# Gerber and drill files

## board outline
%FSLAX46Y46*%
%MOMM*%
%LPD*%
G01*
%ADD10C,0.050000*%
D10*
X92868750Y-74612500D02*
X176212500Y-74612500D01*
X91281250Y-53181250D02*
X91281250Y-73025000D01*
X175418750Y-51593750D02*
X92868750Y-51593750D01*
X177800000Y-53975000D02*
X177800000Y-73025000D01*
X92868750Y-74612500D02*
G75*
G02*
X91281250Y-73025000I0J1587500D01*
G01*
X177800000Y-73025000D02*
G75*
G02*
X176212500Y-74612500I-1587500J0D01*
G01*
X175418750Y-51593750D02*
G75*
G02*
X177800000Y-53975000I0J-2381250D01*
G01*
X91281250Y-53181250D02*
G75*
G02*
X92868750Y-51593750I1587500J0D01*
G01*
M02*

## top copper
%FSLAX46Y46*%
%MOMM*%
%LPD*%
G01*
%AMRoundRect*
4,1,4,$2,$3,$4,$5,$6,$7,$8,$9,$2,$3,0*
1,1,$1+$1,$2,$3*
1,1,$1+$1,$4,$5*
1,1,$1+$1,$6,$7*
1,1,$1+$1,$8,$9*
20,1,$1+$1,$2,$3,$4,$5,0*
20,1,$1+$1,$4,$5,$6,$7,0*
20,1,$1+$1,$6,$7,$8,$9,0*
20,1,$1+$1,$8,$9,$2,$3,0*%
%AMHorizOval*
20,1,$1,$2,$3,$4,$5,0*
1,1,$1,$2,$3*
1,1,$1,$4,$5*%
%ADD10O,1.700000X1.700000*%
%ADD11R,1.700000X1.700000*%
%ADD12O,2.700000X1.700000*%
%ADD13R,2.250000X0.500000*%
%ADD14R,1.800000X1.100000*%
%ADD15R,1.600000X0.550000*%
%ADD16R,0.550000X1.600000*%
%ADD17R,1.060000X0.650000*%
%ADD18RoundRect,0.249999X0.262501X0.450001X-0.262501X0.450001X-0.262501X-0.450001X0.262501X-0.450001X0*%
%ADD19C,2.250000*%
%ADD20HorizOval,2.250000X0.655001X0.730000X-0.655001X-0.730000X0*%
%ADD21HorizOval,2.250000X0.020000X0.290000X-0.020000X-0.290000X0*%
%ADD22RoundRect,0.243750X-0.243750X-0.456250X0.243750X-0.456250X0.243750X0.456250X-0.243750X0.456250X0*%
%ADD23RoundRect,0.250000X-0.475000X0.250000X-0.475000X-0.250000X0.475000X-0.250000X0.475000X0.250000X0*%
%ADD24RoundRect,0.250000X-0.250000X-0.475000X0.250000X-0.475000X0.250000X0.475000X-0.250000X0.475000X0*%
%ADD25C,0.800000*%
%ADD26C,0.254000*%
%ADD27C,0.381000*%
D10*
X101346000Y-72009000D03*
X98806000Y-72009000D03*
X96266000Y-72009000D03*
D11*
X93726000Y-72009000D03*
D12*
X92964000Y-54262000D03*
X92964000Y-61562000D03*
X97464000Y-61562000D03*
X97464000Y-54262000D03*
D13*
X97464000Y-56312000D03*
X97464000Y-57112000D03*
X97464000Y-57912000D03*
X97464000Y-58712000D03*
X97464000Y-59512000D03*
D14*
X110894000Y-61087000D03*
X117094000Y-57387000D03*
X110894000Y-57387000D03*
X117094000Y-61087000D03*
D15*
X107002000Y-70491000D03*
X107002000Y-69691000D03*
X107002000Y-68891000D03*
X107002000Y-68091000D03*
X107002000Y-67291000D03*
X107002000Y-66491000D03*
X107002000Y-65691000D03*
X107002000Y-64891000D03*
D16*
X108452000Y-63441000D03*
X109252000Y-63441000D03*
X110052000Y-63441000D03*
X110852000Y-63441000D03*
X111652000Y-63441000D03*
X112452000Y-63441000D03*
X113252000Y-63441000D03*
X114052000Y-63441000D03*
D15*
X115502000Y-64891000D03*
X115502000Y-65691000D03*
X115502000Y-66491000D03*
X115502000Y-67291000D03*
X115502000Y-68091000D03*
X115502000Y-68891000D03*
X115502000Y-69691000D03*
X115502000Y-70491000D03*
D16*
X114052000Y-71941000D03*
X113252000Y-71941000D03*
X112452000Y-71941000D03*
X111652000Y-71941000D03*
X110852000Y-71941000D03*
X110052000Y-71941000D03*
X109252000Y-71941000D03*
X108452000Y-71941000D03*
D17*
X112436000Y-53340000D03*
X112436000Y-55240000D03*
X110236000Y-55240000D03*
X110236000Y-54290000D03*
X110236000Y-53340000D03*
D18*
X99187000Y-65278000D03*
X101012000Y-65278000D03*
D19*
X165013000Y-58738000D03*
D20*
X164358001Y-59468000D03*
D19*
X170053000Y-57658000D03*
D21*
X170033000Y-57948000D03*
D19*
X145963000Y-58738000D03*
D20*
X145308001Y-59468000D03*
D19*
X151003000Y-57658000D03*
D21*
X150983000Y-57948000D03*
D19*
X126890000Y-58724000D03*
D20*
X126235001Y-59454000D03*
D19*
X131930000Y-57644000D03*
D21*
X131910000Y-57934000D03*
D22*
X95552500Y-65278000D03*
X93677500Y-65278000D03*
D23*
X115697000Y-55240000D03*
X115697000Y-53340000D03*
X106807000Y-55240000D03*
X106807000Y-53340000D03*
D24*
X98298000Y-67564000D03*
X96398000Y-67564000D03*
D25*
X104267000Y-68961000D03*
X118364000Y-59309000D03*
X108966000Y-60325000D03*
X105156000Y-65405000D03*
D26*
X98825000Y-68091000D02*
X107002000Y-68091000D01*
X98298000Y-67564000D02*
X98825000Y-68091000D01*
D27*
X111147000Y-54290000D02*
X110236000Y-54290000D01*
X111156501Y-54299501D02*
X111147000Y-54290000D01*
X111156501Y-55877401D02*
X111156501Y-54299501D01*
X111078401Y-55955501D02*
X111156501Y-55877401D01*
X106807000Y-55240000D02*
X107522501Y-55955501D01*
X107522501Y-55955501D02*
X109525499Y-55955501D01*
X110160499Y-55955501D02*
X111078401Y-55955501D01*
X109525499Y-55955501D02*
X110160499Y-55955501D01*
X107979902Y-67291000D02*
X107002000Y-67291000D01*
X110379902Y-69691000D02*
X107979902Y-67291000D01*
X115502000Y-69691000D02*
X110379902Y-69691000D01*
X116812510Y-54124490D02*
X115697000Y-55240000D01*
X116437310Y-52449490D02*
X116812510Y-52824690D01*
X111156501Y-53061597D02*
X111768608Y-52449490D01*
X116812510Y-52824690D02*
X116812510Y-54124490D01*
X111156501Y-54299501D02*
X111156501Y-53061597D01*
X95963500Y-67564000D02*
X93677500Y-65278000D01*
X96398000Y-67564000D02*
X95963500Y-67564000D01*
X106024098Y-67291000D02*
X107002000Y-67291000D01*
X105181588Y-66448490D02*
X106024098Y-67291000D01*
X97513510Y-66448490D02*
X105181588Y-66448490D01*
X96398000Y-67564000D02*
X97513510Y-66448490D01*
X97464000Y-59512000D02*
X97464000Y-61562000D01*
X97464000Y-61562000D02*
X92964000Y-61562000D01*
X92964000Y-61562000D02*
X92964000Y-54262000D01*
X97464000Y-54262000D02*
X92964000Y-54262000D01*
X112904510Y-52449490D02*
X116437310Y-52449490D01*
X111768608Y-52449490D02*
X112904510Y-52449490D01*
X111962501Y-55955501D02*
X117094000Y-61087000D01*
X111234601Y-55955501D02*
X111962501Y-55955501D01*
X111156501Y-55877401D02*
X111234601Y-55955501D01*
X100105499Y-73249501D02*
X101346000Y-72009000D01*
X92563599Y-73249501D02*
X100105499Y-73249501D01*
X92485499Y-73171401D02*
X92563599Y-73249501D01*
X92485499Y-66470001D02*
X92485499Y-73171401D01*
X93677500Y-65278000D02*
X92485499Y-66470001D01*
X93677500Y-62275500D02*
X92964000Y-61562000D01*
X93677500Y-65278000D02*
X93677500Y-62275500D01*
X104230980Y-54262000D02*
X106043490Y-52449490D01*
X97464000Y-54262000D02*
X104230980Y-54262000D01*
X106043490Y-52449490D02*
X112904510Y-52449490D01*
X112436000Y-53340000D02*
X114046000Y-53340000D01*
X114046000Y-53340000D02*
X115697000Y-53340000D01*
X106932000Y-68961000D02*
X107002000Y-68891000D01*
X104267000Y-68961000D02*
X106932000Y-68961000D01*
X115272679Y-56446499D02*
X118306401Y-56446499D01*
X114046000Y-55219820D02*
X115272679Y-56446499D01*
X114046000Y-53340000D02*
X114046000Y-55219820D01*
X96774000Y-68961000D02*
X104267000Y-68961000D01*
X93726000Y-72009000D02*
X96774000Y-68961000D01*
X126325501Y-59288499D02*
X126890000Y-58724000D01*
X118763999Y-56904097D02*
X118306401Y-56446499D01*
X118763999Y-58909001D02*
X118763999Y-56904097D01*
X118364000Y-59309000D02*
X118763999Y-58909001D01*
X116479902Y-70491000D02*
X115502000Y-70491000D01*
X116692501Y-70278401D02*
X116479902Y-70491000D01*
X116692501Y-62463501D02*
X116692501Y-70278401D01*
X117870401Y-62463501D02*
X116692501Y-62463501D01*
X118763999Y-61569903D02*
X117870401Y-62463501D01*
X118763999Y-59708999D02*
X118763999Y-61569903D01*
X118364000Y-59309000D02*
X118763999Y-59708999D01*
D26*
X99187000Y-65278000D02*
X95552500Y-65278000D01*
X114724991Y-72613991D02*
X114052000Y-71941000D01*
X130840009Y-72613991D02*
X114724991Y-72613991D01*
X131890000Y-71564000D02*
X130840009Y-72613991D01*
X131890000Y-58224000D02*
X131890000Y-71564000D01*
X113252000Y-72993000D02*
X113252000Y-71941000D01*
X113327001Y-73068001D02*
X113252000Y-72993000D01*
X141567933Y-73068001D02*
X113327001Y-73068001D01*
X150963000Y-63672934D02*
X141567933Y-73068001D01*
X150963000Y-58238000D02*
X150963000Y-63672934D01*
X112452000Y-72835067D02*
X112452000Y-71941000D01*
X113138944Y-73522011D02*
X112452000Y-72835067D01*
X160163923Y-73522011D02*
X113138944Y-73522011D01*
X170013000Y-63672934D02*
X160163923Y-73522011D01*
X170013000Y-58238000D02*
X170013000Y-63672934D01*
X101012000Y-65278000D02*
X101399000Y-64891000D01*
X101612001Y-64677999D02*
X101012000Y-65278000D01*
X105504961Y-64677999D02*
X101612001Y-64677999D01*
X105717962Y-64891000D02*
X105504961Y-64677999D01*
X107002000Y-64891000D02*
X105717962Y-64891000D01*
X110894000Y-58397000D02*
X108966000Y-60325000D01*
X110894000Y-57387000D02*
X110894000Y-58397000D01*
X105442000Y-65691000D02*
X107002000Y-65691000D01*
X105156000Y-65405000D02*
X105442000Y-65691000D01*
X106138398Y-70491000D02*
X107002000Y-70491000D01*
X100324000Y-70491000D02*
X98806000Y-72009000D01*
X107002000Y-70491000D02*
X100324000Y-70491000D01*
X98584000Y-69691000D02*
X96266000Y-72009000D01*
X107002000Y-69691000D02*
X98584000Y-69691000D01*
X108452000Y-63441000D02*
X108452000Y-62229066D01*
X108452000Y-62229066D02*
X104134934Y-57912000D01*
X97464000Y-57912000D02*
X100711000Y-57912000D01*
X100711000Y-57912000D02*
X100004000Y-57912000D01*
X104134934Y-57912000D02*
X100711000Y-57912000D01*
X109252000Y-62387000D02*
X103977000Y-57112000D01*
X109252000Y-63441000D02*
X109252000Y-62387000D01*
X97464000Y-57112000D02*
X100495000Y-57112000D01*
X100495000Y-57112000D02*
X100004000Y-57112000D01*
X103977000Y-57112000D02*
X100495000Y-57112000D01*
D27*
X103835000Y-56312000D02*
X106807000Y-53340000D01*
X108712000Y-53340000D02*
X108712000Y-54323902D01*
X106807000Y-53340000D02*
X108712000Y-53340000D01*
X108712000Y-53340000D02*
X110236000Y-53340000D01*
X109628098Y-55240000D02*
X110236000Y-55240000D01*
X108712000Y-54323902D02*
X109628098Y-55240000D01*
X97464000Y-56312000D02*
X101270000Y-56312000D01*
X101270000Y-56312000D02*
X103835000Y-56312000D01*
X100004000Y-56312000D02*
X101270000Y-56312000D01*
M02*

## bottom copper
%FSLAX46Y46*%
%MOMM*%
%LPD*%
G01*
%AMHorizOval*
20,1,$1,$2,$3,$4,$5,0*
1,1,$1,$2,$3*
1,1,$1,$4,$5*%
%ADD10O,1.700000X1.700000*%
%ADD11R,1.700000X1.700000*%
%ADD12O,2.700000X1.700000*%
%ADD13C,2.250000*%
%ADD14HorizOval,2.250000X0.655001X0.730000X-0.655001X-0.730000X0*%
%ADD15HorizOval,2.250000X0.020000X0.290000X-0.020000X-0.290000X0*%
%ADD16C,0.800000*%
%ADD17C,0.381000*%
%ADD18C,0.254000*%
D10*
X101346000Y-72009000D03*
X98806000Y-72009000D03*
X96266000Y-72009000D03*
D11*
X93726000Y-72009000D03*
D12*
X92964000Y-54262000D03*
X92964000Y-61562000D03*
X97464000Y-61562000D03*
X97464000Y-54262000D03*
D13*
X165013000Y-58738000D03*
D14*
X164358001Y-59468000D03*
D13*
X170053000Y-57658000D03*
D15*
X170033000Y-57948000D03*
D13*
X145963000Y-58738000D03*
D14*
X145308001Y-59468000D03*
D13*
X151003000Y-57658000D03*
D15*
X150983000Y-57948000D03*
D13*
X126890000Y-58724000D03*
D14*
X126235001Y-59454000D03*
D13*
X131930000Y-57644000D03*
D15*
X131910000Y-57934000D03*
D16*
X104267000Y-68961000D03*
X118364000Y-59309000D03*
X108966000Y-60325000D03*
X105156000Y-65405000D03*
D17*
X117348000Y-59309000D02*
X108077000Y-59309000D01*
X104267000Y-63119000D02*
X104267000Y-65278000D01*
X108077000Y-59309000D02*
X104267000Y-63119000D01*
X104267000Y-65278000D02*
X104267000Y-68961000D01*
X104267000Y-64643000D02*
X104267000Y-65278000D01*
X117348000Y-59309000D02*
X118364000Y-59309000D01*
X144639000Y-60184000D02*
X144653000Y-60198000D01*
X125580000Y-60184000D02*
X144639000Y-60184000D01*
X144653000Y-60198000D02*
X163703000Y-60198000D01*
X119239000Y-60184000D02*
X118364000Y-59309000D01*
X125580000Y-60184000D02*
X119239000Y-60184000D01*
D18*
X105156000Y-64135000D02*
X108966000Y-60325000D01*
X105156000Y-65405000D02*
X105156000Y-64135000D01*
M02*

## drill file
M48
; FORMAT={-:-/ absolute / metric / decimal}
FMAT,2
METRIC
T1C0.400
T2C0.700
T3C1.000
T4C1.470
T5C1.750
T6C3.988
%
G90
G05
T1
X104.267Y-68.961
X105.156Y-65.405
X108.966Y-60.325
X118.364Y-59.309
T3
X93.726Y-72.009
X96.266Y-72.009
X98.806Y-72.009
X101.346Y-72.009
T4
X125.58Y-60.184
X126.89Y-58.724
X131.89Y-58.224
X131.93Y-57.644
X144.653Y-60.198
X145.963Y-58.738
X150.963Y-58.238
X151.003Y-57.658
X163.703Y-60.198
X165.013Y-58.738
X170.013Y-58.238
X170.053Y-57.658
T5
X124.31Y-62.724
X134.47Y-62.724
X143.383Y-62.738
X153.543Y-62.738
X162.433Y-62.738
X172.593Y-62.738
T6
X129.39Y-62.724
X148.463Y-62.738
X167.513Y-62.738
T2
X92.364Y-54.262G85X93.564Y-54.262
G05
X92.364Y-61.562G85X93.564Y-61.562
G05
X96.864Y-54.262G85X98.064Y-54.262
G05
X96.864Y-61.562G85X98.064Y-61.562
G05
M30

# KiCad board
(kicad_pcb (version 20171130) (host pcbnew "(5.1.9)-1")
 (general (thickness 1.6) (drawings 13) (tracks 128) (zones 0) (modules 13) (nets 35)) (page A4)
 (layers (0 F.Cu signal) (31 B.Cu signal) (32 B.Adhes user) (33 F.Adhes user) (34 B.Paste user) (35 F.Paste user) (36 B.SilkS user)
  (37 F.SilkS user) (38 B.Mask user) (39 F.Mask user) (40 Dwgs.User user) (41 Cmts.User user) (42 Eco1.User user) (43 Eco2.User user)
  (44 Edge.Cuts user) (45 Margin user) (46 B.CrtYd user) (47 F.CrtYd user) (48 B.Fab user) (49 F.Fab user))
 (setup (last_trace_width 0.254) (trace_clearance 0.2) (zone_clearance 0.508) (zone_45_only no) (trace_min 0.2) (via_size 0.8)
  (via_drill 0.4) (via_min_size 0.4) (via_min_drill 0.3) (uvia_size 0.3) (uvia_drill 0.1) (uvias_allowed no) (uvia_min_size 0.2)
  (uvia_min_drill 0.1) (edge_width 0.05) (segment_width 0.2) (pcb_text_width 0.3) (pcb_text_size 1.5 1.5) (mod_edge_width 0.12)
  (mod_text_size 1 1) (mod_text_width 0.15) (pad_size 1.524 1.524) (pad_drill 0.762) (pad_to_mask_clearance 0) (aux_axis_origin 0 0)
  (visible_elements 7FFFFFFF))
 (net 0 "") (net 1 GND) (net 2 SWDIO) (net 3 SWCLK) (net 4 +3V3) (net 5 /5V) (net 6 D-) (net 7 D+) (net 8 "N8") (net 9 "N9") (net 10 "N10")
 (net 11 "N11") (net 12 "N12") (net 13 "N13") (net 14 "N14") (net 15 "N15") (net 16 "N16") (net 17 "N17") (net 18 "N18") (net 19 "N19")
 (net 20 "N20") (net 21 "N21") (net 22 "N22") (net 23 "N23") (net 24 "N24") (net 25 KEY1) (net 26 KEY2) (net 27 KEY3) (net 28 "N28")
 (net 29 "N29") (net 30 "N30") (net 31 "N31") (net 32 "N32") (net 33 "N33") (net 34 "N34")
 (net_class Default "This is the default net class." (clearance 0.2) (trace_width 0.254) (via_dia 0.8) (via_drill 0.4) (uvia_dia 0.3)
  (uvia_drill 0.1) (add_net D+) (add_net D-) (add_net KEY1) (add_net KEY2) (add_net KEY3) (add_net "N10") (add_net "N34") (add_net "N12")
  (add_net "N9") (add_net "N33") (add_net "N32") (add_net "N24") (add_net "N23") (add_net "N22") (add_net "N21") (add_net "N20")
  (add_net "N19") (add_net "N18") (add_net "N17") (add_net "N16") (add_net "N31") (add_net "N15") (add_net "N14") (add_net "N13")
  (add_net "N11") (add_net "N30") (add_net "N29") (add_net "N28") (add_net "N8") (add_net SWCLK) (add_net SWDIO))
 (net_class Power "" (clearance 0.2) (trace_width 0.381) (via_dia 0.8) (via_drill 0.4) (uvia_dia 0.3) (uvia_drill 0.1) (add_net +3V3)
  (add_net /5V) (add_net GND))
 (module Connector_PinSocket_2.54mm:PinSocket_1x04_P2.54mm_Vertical (layer F.Cu) (at 93.726 72.009 90)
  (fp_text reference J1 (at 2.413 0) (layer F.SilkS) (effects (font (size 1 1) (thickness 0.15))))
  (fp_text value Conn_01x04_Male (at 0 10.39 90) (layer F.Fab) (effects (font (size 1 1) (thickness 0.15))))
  (pad 4 thru_hole oval (at 0 7.62 90) (size 1.7 1.7) (drill 1) (layers *.Cu *.Mask) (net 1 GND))
  (pad 3 thru_hole oval (at 0 5.08 90) (size 1.7 1.7) (drill 1) (layers *.Cu *.Mask) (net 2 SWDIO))
  (pad 2 thru_hole oval (at 0 2.54 90) (size 1.7 1.7) (drill 1) (layers *.Cu *.Mask) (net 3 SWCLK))
  (pad 1 thru_hole rect (at 0 0 90) (size 1.7 1.7) (drill 1) (layers *.Cu *.Mask) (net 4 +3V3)))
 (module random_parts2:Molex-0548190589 (layer F.Cu) (at 92.964 57.912)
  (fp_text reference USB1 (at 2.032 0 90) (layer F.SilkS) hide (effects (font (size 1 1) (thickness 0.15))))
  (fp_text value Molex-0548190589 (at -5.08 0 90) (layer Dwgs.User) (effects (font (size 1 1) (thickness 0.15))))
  (pad 6 thru_hole oval (at 0 -3.65) (size 2.7 1.7) (drill oval 1.9 0.7) (layers *.Cu *.Mask) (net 1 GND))
  (pad 6 thru_hole oval (at 0 3.65) (size 2.7 1.7) (drill oval 1.9 0.7) (layers *.Cu *.Mask) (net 1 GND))
  (pad 6 thru_hole oval (at 4.5 3.65) (size 2.7 1.7) (drill oval 1.9 0.7) (layers *.Cu *.Mask) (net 1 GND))
  (pad 6 thru_hole oval (at 4.5 -3.65) (size 2.7 1.7) (drill oval 1.9 0.7) (layers *.Cu *.Mask) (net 1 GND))
  (pad 5 smd rect (at 4.5 -1.6) (size 2.25 0.5) (layers F.Cu F.Paste F.Mask) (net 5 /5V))
  (pad 4 smd rect (at 4.5 -0.8) (size 2.25 0.5) (layers F.Cu F.Paste F.Mask) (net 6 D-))
  (pad 3 smd rect (at 4.5 0) (size 2.25 0.5) (layers F.Cu F.Paste F.Mask) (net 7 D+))
  (pad 2 smd rect (at 4.5 0.8) (size 2.25 0.5) (layers F.Cu F.Paste F.Mask) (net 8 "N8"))
  (pad 1 smd rect (at 4.5 1.6) (size 2.25 0.5) (layers F.Cu F.Paste F.Mask) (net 1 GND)))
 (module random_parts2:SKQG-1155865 (layer F.Cu) (at 113.994 59.237)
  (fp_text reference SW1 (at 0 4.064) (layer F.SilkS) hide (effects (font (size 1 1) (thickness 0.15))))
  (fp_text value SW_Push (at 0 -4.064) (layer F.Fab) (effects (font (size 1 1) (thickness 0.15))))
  (pad 4 smd rect (at -3.1 1.85) (size 1.8 1.1) (layers F.Cu F.Paste F.Mask))
  (pad 3 smd rect (at 3.1 -1.85) (size 1.8 1.1) (layers F.Cu F.Paste F.Mask))
  (pad 2 smd rect (at -3.1 -1.85) (size 1.8 1.1) (layers F.Cu F.Paste F.Mask) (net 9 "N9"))
  (pad 1 smd rect (at 3.1 1.85) (size 1.8 1.1) (layers F.Cu F.Paste F.Mask) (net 1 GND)))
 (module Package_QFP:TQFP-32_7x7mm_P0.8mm (layer F.Cu) (at 111.252 67.691 90)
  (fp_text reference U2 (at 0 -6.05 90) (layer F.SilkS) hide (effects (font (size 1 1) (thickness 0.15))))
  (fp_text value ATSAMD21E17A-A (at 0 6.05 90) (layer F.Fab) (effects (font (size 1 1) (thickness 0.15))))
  (pad 32 smd rect (at -2.8 -4.25 180) (size 1.6 0.55) (layers F.Cu F.Paste F.Mask) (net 2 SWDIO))
  (pad 31 smd rect (at -2 -4.25 180) (size 1.6 0.55) (layers F.Cu F.Paste F.Mask) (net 3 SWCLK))
  (pad 30 smd rect (at -1.2 -4.25 180) (size 1.6 0.55) (layers F.Cu F.Paste F.Mask) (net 4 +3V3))
  (pad 29 smd rect (at -0.4 -4.25 180) (size 1.6 0.55) (layers F.Cu F.Paste F.Mask) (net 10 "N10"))
  (pad 28 smd rect (at 0.4 -4.25 180) (size 1.6 0.55) (layers F.Cu F.Paste F.Mask) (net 1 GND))
  (pad 27 smd rect (at 1.2 -4.25 180) (size 1.6 0.55) (layers F.Cu F.Paste F.Mask) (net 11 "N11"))
  (pad 26 smd rect (at 2 -4.25 180) (size 1.6 0.55) (layers F.Cu F.Paste F.Mask) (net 9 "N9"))
  (pad 25 smd rect (at 2.8 -4.25 180) (size 1.6 0.55) (layers F.Cu F.Paste F.Mask) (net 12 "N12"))
  (pad 24 smd rect (at 4.25 -2.8 90) (size 1.6 0.55) (layers F.Cu F.Paste F.Mask) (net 7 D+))
  (pad 23 smd rect (at 4.25 -2 90) (size 1.6 0.55) (layers F.Cu F.Paste F.Mask) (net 6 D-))
  (pad 22 smd rect (at 4.25 -1.2 90) (size 1.6 0.55) (layers F.Cu F.Paste F.Mask) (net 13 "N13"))
  (pad 21 smd rect (at 4.25 -0.4 90) (size 1.6 0.55) (layers F.Cu F.Paste F.Mask) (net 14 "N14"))
  (pad 20 smd rect (at 4.25 0.4 90) (size 1.6 0.55) (layers F.Cu F.Paste F.Mask) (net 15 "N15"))
  (pad 19 smd rect (at 4.25 1.2 90) (size 1.6 0.55) (layers F.Cu F.Paste F.Mask) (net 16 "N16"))
  (pad 18 smd rect (at 4.25 2 90) (size 1.6 0.55) (layers F.Cu F.Paste F.Mask) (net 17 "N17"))
  (pad 17 smd rect (at 4.25 2.8 90) (size 1.6 0.55) (layers F.Cu F.Paste F.Mask) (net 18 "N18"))
  (pad 16 smd rect (at 2.8 4.25 180) (size 1.6 0.55) (layers F.Cu F.Paste F.Mask) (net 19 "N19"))
  (pad 15 smd rect (at 2 4.25 180) (size 1.6 0.55) (layers F.Cu F.Paste F.Mask) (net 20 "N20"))
  (pad 14 smd rect (at 1.2 4.25 180) (size 1.6 0.55) (layers F.Cu F.Paste F.Mask) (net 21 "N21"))
  (pad 13 smd rect (at 0.4 4.25 180) (size 1.6 0.55) (layers F.Cu F.Paste F.Mask) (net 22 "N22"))
  (pad 12 smd rect (at -0.4 4.25 180) (size 1.6 0.55) (layers F.Cu F.Paste F.Mask) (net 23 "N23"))
  (pad 11 smd rect (at -1.2 4.25 180) (size 1.6 0.55) (layers F.Cu F.Paste F.Mask) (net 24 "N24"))
  (pad 10 smd rect (at -2 4.25 180) (size 1.6 0.55) (layers F.Cu F.Paste F.Mask) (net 1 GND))
  (pad 9 smd rect (at -2.8 4.25 180) (size 1.6 0.55) (layers F.Cu F.Paste F.Mask) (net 4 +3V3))
  (pad 8 smd rect (at -4.25 2.8 90) (size 1.6 0.55) (layers F.Cu F.Paste F.Mask) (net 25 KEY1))
  (pad 7 smd rect (at -4.25 2 90) (size 1.6 0.55) (layers F.Cu F.Paste F.Mask) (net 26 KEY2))
  (pad 6 smd rect (at -4.25 1.2 90) (size 1.6 0.55) (layers F.Cu F.Paste F.Mask) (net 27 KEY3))
  (pad 5 smd rect (at -4.25 0.4 90) (size 1.6 0.55) (layers F.Cu F.Paste F.Mask) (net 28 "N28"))
  (pad 4 smd rect (at -4.25 -0.4 90) (size 1.6 0.55) (layers F.Cu F.Paste F.Mask) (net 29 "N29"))
  (pad 3 smd rect (at -4.25 -1.2 90) (size 1.6 0.55) (layers F.Cu F.Paste F.Mask) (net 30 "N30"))
  (pad 2 smd rect (at -4.25 -2 90) (size 1.6 0.55) (layers F.Cu F.Paste F.Mask) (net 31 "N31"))
  (pad 1 smd rect (at -4.25 -2.8 90) (size 1.6 0.55) (layers F.Cu F.Paste F.Mask) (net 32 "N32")))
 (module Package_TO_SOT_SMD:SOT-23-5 (layer F.Cu) (at 111.336 54.29)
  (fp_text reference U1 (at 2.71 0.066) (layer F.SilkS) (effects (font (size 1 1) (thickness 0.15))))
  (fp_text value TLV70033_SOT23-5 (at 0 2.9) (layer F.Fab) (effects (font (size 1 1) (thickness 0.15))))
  (pad 5 smd rect (at 1.1 -0.95) (size 1.06 0.65) (layers F.Cu F.Paste F.Mask) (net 4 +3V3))
  (pad 4 smd rect (at 1.1 0.95) (size 1.06 0.65) (layers F.Cu F.Paste F.Mask) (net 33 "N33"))
  (pad 3 smd rect (at -1.1 0.95) (size 1.06 0.65) (layers F.Cu F.Paste F.Mask) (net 5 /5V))
  (pad 2 smd rect (at -1.1 0) (size 1.06 0.65) (layers F.Cu F.Paste F.Mask) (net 1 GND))
  (pad 1 smd rect (at -1.1 -0.95) (size 1.06 0.65) (layers F.Cu F.Paste F.Mask) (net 5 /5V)))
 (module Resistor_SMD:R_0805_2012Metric (layer F.Cu) (at 100.0995 65.278 180)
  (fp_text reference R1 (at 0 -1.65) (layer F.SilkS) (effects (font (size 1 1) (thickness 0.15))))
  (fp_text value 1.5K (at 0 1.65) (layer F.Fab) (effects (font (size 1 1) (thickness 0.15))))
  (pad 2 smd roundrect (at 0.9125 0 180) (size 1.025 1.4) (layers F.Cu F.Paste F.Mask) (roundrect_rratio 0.2439014634146341) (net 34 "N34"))
  (pad 1 smd roundrect (at -0.9125 0 180) (size 1.025 1.4) (layers F.Cu F.Paste F.Mask) (roundrect_rratio 0.2439014634146341) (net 12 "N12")))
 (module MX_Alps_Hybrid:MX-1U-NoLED (layer F.Cu) (at 167.513 62.738)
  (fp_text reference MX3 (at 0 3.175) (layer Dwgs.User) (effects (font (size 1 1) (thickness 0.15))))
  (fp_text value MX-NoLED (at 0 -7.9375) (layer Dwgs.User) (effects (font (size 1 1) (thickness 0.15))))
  (pad "" np_thru_hole circle (at 5.08 0 48.0996) (size 1.75 1.75) (drill 1.75) (layers *.Cu *.Mask))
  (pad "" np_thru_hole circle (at -5.08 0 48.0996) (size 1.75 1.75) (drill 1.75) (layers *.Cu *.Mask))
  (pad 1 thru_hole circle (at -2.5 -4) (size 2.25 2.25) (drill 1.47) (layers *.Cu B.Mask) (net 4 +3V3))
  (pad "" np_thru_hole circle (at 0 0) (size 3.9878 3.9878) (drill 3.9878) (layers *.Cu *.Mask))
  (pad 1 thru_hole oval (at -3.81 -2.54 48.0996) (size 4.211556 2.25) (drill 1.47 (offset 0.980778 0)) (layers *.Cu B.Mask) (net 4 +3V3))
  (pad 2 thru_hole circle (at 2.54 -5.08) (size 2.25 2.25) (drill 1.47) (layers *.Cu B.Mask) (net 27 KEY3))
  (pad 2 thru_hole oval (at 2.5 -4.5 86.0548) (size 2.831378 2.25) (drill 1.47 (offset 0.290689 0)) (layers *.Cu B.Mask) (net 27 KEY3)))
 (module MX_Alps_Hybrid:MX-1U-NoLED (layer F.Cu) (at 148.463 62.738)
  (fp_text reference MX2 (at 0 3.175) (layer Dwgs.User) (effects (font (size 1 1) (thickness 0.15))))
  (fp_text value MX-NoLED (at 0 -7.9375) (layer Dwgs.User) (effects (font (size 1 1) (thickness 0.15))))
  (pad "" np_thru_hole circle (at 5.08 0 48.0996) (size 1.75 1.75) (drill 1.75) (layers *.Cu *.Mask))
  (pad "" np_thru_hole circle (at -5.08 0 48.0996) (size 1.75 1.75) (drill 1.75) (layers *.Cu *.Mask))
  (pad 1 thru_hole circle (at -2.5 -4) (size 2.25 2.25) (drill 1.47) (layers *.Cu B.Mask) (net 4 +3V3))
  (pad "" np_thru_hole circle (at 0 0) (size 3.9878 3.9878) (drill 3.9878) (layers *.Cu *.Mask))
  (pad 1 thru_hole oval (at -3.81 -2.54 48.0996) (size 4.211556 2.25) (drill 1.47 (offset 0.980778 0)) (layers *.Cu B.Mask) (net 4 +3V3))
  (pad 2 thru_hole circle (at 2.54 -5.08) (size 2.25 2.25) (drill 1.47) (layers *.Cu B.Mask) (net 26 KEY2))
  (pad 2 thru_hole oval (at 2.5 -4.5 86.0548) (size 2.831378 2.25) (drill 1.47 (offset 0.290689 0)) (layers *.Cu B.Mask) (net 26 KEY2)))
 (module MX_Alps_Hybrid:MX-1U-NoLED (layer F.Cu) (at 129.39 62.724)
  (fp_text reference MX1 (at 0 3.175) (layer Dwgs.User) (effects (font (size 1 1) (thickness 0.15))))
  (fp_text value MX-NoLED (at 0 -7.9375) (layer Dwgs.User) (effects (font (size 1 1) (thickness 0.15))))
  (pad "" np_thru_hole circle (at 5.08 0 48.0996) (size 1.75 1.75) (drill 1.75) (layers *.Cu *.Mask))
  (pad "" np_thru_hole circle (at -5.08 0 48.0996) (size 1.75 1.75) (drill 1.75) (layers *.Cu *.Mask))
  (pad 1 thru_hole circle (at -2.5 -4) (size 2.25 2.25) (drill 1.47) (layers *.Cu B.Mask) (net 4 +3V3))
  (pad "" np_thru_hole circle (at 0 0) (size 3.9878 3.9878) (drill 3.9878) (layers *.Cu *.Mask))
  (pad 1 thru_hole oval (at -3.81 -2.54 48.0996) (size 4.211556 2.25) (drill 1.47 (offset 0.980778 0)) (layers *.Cu B.Mask) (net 4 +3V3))
  (pad 2 thru_hole circle (at 2.54 -5.08) (size 2.25 2.25) (drill 1.47) (layers *.Cu B.Mask) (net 25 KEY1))
  (pad 2 thru_hole oval (at 2.5 -4.5 86.0548) (size 2.831378 2.25) (drill 1.47 (offset 0.290689 0)) (layers *.Cu B.Mask) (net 25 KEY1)))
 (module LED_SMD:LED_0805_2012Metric (layer F.Cu) (at 94.615 65.278)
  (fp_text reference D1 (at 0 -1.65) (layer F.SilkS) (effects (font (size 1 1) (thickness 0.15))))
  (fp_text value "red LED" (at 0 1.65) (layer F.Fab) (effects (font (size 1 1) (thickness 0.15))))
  (pad 2 smd roundrect (at 0.9375 0) (size 0.975 1.4) (layers F.Cu F.Paste F.Mask) (roundrect_rratio 0.25) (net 34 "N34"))
  (pad 1 smd roundrect (at -0.9375 0) (size 0.975 1.4) (layers F.Cu F.Paste F.Mask) (roundrect_rratio 0.25) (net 1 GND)))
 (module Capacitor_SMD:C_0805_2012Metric (layer F.Cu) (at 115.697 54.29 270)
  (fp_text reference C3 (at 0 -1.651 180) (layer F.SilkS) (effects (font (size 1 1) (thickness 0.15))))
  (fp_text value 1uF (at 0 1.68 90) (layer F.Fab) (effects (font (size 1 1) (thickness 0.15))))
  (pad 2 smd roundrect (at 0.95 0 270) (size 1 1.45) (layers F.Cu F.Paste F.Mask) (roundrect_rratio 0.25) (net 1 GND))
  (pad 1 smd roundrect (at -0.95 0 270) (size 1 1.45) (layers F.Cu F.Paste F.Mask) (roundrect_rratio 0.25) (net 4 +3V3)))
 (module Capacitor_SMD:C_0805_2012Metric (layer F.Cu) (at 106.807 54.29 270)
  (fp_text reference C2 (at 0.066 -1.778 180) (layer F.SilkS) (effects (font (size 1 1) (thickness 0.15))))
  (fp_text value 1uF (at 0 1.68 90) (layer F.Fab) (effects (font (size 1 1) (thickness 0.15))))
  (pad 2 smd roundrect (at 0.95 0 270) (size 1 1.45) (layers F.Cu F.Paste F.Mask) (roundrect_rratio 0.25) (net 1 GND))
  (pad 1 smd roundrect (at -0.95 0 270) (size 1 1.45) (layers F.Cu F.Paste F.Mask) (roundrect_rratio 0.25) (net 5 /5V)))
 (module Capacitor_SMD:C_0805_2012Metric (layer F.Cu) (at 97.348 67.564)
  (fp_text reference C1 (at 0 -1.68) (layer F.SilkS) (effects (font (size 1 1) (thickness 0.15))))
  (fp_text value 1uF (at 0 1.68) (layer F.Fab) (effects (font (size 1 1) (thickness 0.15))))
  (pad 2 smd roundrect (at 0.95 0) (size 1 1.45) (layers F.Cu F.Paste F.Mask) (roundrect_rratio 0.25) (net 10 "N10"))
  (pad 1 smd roundrect (at -0.95 0) (size 1 1.45) (layers F.Cu F.Paste F.Mask) (roundrect_rratio 0.25) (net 1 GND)))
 (gr_line (start 92.86875 74.6125) (end 176.2125 74.6125) (layer Edge.Cuts) (width 0.05))
 (gr_line (start 91.28125 53.18125) (end 91.28125 73.025) (layer Edge.Cuts) (width 0.05))
 (gr_line (start 175.41875 51.59375) (end 92.86875 51.59375) (layer Edge.Cuts) (width 0.05))
 (gr_line (start 177.8 53.975) (end 177.8 73.025) (layer Edge.Cuts) (width 0.05))
 (gr_arc (start 92.86875 73.025) (end 91.28125 73.025) (angle -90) (layer Edge.Cuts) (width 0.05))
 (gr_arc (start 176.2125 73.025) (end 176.2125 74.6125) (angle -90) (layer Edge.Cuts) (width 0.05))
 (gr_arc (start 175.41875 53.975) (end 177.8 53.975) (angle -90) (layer Edge.Cuts) (width 0.05))
 (gr_arc (start 92.86875 53.18125) (end 92.86875 51.59375) (angle -90) (layer Edge.Cuts) (width 0.05))
 (segment (start 98.825 68.091) (end 107.002 68.091) (width 0.254) (layer F.Cu) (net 10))
 (segment (start 98.298 67.564) (end 98.825 68.091) (width 0.254) (layer F.Cu) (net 10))
 (segment (start 111.147 54.29) (end 110.236 54.29) (width 0.381) (layer F.Cu) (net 1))
 (segment (start 111.156501 54.299501) (end 111.147 54.29) (width 0.381) (layer F.Cu) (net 1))
 (segment (start 111.156501 55.877401) (end 111.156501 54.299501) (width 0.381) (layer F.Cu) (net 1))
 (segment (start 111.078401 55.955501) (end 111.156501 55.877401) (width 0.381) (layer F.Cu) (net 1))
 (segment (start 106.807 55.24) (end 107.522501 55.955501) (width 0.381) (layer F.Cu) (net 1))
 (segment (start 107.522501 55.955501) (end 109.525499 55.955501) (width 0.381) (layer F.Cu) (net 1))
 (segment (start 110.160499 55.955501) (end 111.078401 55.955501) (width 0.381) (layer F.Cu) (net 1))
 (segment (start 109.525499 55.955501) (end 110.160499 55.955501) (width 0.381) (layer F.Cu) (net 1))
 (segment (start 107.979902 67.291) (end 107.002 67.291) (width 0.381) (layer F.Cu) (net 1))
 (segment (start 110.379902 69.691) (end 107.979902 67.291) (width 0.381) (layer F.Cu) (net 1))
 (segment (start 115.502 69.691) (end 110.379902 69.691) (width 0.381) (layer F.Cu) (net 1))
 (segment (start 116.81251 54.12449) (end 115.697 55.24) (width 0.381) (layer F.Cu) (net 1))
 (segment (start 116.43731 52.44949) (end 116.81251 52.82469) (width 0.381) (layer F.Cu) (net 1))
 (segment (start 111.156501 53.061597) (end 111.768608 52.44949) (width 0.381) (layer F.Cu) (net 1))
 (segment (start 116.81251 52.82469) (end 116.81251 54.12449) (width 0.381) (layer F.Cu) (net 1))
 (segment (start 111.156501 54.299501) (end 111.156501 53.061597) (width 0.381) (layer F.Cu) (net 1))
 (segment (start 95.9635 67.564) (end 93.6775 65.278) (width 0.381) (layer F.Cu) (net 1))
 (segment (start 96.398 67.564) (end 95.9635 67.564) (width 0.381) (layer F.Cu) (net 1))
 (segment (start 106.024098 67.291) (end 107.002 67.291) (width 0.381) (layer F.Cu) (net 1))
 (segment (start 105.181588 66.44849) (end 106.024098 67.291) (width 0.381) (layer F.Cu) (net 1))
 (segment (start 97.51351 66.44849) (end 105.181588 66.44849) (width 0.381) (layer F.Cu) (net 1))
 (segment (start 96.398 67.564) (end 97.51351 66.44849) (width 0.381) (layer F.Cu) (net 1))
 (segment (start 97.464 59.512) (end 97.464 61.562) (width 0.381) (layer F.Cu) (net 1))
 (segment (start 97.464 61.562) (end 92.964 61.562) (width 0.381) (layer F.Cu) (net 1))
 (segment (start 92.964 61.562) (end 92.964 54.262) (width 0.381) (layer F.Cu) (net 1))
 (segment (start 97.464 54.262) (end 92.964 54.262) (width 0.381) (layer F.Cu) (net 1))
 (segment (start 112.90451 52.44949) (end 116.43731 52.44949) (width 0.381) (layer F.Cu) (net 1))
 (segment (start 111.768608 52.44949) (end 112.90451 52.44949) (width 0.381) (layer F.Cu) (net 1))
 (segment (start 111.962501 55.955501) (end 117.094 61.087) (width 0.381) (layer F.Cu) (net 1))
 (segment (start 111.234601 55.955501) (end 111.962501 55.955501) (width 0.381) (layer F.Cu) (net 1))
 (segment (start 111.156501 55.877401) (end 111.234601 55.955501) (width 0.381) (layer F.Cu) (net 1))
 (segment (start 100.105499 73.249501) (end 101.346 72.009) (width 0.381) (layer F.Cu) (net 1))
 (segment (start 92.563599 73.249501) (end 100.105499 73.249501) (width 0.381) (layer F.Cu) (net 1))
 (segment (start 92.485499 73.171401) (end 92.563599 73.249501) (width 0.381) (layer F.Cu) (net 1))
 (segment (start 92.485499 66.470001) (end 92.485499 73.171401) (width 0.381) (layer F.Cu) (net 1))
 (segment (start 93.6775 65.278) (end 92.485499 66.470001) (width 0.381) (layer F.Cu) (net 1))
 (segment (start 93.6775 62.2755) (end 92.964 61.562) (width 0.381) (layer F.Cu) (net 1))
 (segment (start 93.6775 65.278) (end 93.6775 62.2755) (width 0.381) (layer F.Cu) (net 1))
 (segment (start 104.23098 54.262) (end 106.04349 52.44949) (width 0.381) (layer F.Cu) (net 1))
 (segment (start 97.464 54.262) (end 104.23098 54.262) (width 0.381) (layer F.Cu) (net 1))
 (segment (start 106.04349 52.44949) (end 112.90451 52.44949) (width 0.381) (layer F.Cu) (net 1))
 (segment (start 112.436 53.34) (end 114.046 53.34) (width 0.381) (layer F.Cu) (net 4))
 (segment (start 114.046 53.34) (end 115.697 53.34) (width 0.381) (layer F.Cu) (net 4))
 (via (at 104.267 68.961) (size 0.8) (drill 0.4) (layers F.Cu B.Cu) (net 4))
 (segment (start 106.932 68.961) (end 107.002 68.891) (width 0.381) (layer F.Cu) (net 4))
 (segment (start 104.267 68.961) (end 106.932 68.961) (width 0.381) (layer F.Cu) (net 4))
 (segment (start 115.272679 56.446499) (end 118.306401 56.446499) (width 0.381) (layer F.Cu) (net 4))
 (segment (start 114.046 55.21982) (end 115.272679 56.446499) (width 0.381) (layer F.Cu) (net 4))
 (segment (start 114.046 53.34) (end 114.046 55.21982) (width 0.381) (layer F.Cu) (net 4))
 (segment (start 117.348 59.309) (end 108.077 59.309) (width 0.381) (layer B.Cu) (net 4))
 (segment (start 104.267 63.119) (end 104.267 65.278) (width 0.381) (layer B.Cu) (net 4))
 (segment (start 108.077 59.309) (end 104.267 63.119) (width 0.381) (layer B.Cu) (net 4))
 (segment (start 104.267 65.278) (end 104.267 68.961) (width 0.381) (layer B.Cu) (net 4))
 (segment (start 104.267 64.643) (end 104.267 65.278) (width 0.381) (layer B.Cu) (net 4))
 (segment (start 96.774 68.961) (end 104.267 68.961) (width 0.381) (layer F.Cu) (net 4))
 (segment (start 93.726 72.009) (end 96.774 68.961) (width 0.381) (layer F.Cu) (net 4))
 (segment (start 126.325501 59.288499) (end 126.89 58.724) (width 0.381) (layer F.Cu) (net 4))
 (via (at 118.364 59.309) (size 0.8) (drill 0.4) (layers F.Cu B.Cu) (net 4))
 (segment (start 117.348 59.309) (end 118.364 59.309) (width 0.381) (layer B.Cu) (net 4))
 (segment (start 118.763999 56.904097) (end 118.306401 56.446499) (width 0.381) (layer F.Cu) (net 4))
 (segment (start 118.763999 58.909001) (end 118.763999 56.904097) (width 0.381) (layer F.Cu) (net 4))
 (segment (start 118.364 59.309) (end 118.763999 58.909001) (width 0.381) (layer F.Cu) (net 4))
 (segment (start 116.479902 70.491) (end 115.502 70.491) (width 0.381) (layer F.Cu) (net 4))
 (segment (start 116.692501 70.278401) (end 116.479902 70.491) (width 0.381) (layer F.Cu) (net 4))
 (segment (start 116.692501 62.463501) (end 116.692501 70.278401) (width 0.381) (layer F.Cu) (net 4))
 (segment (start 117.870401 62.463501) (end 116.692501 62.463501) (width 0.381) (layer F.Cu) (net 4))
 (segment (start 118.763999 61.569903) (end 117.870401 62.463501) (width 0.381) (layer F.Cu) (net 4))
 (segment (start 118.763999 59.708999) (end 118.763999 61.569903) (width 0.381) (layer F.Cu) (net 4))
 (segment (start 118.364 59.309) (end 118.763999 59.708999) (width 0.381) (layer F.Cu) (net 4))
 (segment (start 144.639 60.184) (end 144.653 60.198) (width 0.381) (layer B.Cu) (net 4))
 (segment (start 125.58 60.184) (end 144.639 60.184) (width 0.381) (layer B.Cu) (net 4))
 (segment (start 144.653 60.198) (end 163.703 60.198) (width 0.381) (layer B.Cu) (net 4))
 (segment (start 119.239 60.184) (end 118.364 59.309) (width 0.381) (layer B.Cu) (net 4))
 (segment (start 125.58 60.184) (end 119.239 60.184) (width 0.381) (layer B.Cu) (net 4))
 (segment (start 99.187 65.278) (end 95.5525 65.278) (width 0.254) (layer F.Cu) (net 34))
 (segment (start 114.724991 72.613991) (end 114.052 71.941) (width 0.254) (layer F.Cu) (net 25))
 (segment (start 130.840009 72.613991) (end 114.724991 72.613991) (width 0.254) (layer F.Cu) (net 25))
 (segment (start 131.89 71.564) (end 130.840009 72.613991) (width 0.254) (layer F.Cu) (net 25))
 (segment (start 131.89 58.224) (end 131.89 71.564) (width 0.254) (layer F.Cu) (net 25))
 (segment (start 113.252 72.993) (end 113.252 71.941) (width 0.254) (layer F.Cu) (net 26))
 (segment (start 113.327001 73.068001) (end 113.252 72.993) (width 0.254) (layer F.Cu) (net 26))
 (segment (start 141.567933 73.068001) (end 113.327001 73.068001) (width 0.254) (layer F.Cu) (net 26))
 (segment (start 150.963 63.672934) (end 141.567933 73.068001) (width 0.254) (layer F.Cu) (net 26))
 (segment (start 150.963 58.238) (end 150.963 63.672934) (width 0.254) (layer F.Cu) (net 26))
 (segment (start 112.452 72.835067) (end 112.452 71.941) (width 0.254) (layer F.Cu) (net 27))
 (segment (start 113.138944 73.522011) (end 112.452 72.835067) (width 0.254) (layer F.Cu) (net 27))
 (segment (start 160.163923 73.522011) (end 113.138944 73.522011) (width 0.254) (layer F.Cu) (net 27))
 (segment (start 170.013 63.672934) (end 160.163923 73.522011) (width 0.254) (layer F.Cu) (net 27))
 (segment (start 170.013 58.238) (end 170.013 63.672934) (width 0.254) (layer F.Cu) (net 27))
 (segment (start 101.012 65.278) (end 101.399 64.891) (width 0.254) (layer F.Cu) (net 12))
 (segment (start 101.612001 64.677999) (end 101.012 65.278) (width 0.254) (layer F.Cu) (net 12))
 (segment (start 105.504961 64.677999) (end 101.612001 64.677999) (width 0.254) (layer F.Cu) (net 12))
 (segment (start 105.717962 64.891) (end 105.504961 64.677999) (width 0.254) (layer F.Cu) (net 12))
 (segment (start 107.002 64.891) (end 105.717962 64.891) (width 0.254) (layer F.Cu) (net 12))
 (via (at 108.966 60.325) (size 0.8) (drill 0.4) (layers F.Cu B.Cu) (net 9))
 (segment (start 110.894 58.397) (end 108.966 60.325) (width 0.254) (layer F.Cu) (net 9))
 (segment (start 110.894 57.387) (end 110.894 58.397) (width 0.254) (layer F.Cu) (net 9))
 (via (at 105.156 65.405) (size 0.8) (drill 0.4) (layers F.Cu B.Cu) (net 9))
 (segment (start 105.442 65.691) (end 107.002 65.691) (width 0.254) (layer F.Cu) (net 9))
 (segment (start 105.156 65.405) (end 105.442 65.691) (width 0.254) (layer F.Cu) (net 9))
 (segment (start 105.156 64.135) (end 108.966 60.325) (width 0.254) (layer B.Cu) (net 9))
 (segment (start 105.156 65.405) (end 105.156 64.135) (width 0.254) (layer B.Cu) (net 9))
 (segment (start 106.138398 70.491) (end 107.002 70.491) (width 0.254) (layer F.Cu) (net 2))
 (segment (start 100.324 70.491) (end 98.806 72.009) (width 0.254) (layer F.Cu) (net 2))
 (segment (start 107.002 70.491) (end 100.324 70.491) (width 0.254) (layer F.Cu) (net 2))
 (segment (start 98.584 69.691) (end 96.266 72.009) (width 0.254) (layer F.Cu) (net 3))
 (segment (start 107.002 69.691) (end 98.584 69.691) (width 0.254) (layer F.Cu) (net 3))
 (segment (start 108.452 63.441) (end 108.452 62.229066) (width 0.254) (layer F.Cu) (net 7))
 (segment (start 108.452 62.229066) (end 104.134934 57.912) (width 0.254) (layer F.Cu) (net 7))
 (segment (start 97.464 57.912) (end 100.711 57.912) (width 0.254) (layer F.Cu) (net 7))
 (segment (start 100.711 57.912) (end 100.004 57.912) (width 0.254) (layer F.Cu) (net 7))
 (segment (start 104.134934 57.912) (end 100.711 57.912) (width 0.254) (layer F.Cu) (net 7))
 (segment (start 109.252 62.387) (end 103.977 57.112) (width 0.254) (layer F.Cu) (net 6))
 (segment (start 109.252 63.441) (end 109.252 62.387) (width 0.254) (layer F.Cu) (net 6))
 (segment (start 97.464 57.112) (end 100.495 57.112) (width 0.254) (layer F.Cu) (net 6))
 (segment (start 100.495 57.112) (end 100.004 57.112) (width 0.254) (layer F.Cu) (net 6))
 (segment (start 103.977 57.112) (end 100.495 57.112) (width 0.254) (layer F.Cu) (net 6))
 (segment (start 103.835 56.312) (end 106.807 53.34) (width 0.381) (layer F.Cu) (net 5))
 (segment (start 108.712 53.34) (end 108.712 54.323902) (width 0.381) (layer F.Cu) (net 5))
 (segment (start 106.807 53.34) (end 108.712 53.34) (width 0.381) (layer F.Cu) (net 5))
 (segment (start 108.712 53.34) (end 110.236 53.34) (width 0.381) (layer F.Cu) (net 5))
 (segment (start 109.628098 55.24) (end 110.236 55.24) (width 0.381) (layer F.Cu) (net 5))
 (segment (start 108.712 54.323902) (end 109.628098 55.24) (width 0.381) (layer F.Cu) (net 5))
 (segment (start 97.464 56.312) (end 101.27 56.312) (width 0.381) (layer F.Cu) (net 5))
 (segment (start 101.27 56.312) (end 103.835 56.312) (width 0.381) (layer F.Cu) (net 5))
 (segment (start 100.004 56.312) (end 101.27 56.312) (width 0.381) (layer F.Cu) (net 5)))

